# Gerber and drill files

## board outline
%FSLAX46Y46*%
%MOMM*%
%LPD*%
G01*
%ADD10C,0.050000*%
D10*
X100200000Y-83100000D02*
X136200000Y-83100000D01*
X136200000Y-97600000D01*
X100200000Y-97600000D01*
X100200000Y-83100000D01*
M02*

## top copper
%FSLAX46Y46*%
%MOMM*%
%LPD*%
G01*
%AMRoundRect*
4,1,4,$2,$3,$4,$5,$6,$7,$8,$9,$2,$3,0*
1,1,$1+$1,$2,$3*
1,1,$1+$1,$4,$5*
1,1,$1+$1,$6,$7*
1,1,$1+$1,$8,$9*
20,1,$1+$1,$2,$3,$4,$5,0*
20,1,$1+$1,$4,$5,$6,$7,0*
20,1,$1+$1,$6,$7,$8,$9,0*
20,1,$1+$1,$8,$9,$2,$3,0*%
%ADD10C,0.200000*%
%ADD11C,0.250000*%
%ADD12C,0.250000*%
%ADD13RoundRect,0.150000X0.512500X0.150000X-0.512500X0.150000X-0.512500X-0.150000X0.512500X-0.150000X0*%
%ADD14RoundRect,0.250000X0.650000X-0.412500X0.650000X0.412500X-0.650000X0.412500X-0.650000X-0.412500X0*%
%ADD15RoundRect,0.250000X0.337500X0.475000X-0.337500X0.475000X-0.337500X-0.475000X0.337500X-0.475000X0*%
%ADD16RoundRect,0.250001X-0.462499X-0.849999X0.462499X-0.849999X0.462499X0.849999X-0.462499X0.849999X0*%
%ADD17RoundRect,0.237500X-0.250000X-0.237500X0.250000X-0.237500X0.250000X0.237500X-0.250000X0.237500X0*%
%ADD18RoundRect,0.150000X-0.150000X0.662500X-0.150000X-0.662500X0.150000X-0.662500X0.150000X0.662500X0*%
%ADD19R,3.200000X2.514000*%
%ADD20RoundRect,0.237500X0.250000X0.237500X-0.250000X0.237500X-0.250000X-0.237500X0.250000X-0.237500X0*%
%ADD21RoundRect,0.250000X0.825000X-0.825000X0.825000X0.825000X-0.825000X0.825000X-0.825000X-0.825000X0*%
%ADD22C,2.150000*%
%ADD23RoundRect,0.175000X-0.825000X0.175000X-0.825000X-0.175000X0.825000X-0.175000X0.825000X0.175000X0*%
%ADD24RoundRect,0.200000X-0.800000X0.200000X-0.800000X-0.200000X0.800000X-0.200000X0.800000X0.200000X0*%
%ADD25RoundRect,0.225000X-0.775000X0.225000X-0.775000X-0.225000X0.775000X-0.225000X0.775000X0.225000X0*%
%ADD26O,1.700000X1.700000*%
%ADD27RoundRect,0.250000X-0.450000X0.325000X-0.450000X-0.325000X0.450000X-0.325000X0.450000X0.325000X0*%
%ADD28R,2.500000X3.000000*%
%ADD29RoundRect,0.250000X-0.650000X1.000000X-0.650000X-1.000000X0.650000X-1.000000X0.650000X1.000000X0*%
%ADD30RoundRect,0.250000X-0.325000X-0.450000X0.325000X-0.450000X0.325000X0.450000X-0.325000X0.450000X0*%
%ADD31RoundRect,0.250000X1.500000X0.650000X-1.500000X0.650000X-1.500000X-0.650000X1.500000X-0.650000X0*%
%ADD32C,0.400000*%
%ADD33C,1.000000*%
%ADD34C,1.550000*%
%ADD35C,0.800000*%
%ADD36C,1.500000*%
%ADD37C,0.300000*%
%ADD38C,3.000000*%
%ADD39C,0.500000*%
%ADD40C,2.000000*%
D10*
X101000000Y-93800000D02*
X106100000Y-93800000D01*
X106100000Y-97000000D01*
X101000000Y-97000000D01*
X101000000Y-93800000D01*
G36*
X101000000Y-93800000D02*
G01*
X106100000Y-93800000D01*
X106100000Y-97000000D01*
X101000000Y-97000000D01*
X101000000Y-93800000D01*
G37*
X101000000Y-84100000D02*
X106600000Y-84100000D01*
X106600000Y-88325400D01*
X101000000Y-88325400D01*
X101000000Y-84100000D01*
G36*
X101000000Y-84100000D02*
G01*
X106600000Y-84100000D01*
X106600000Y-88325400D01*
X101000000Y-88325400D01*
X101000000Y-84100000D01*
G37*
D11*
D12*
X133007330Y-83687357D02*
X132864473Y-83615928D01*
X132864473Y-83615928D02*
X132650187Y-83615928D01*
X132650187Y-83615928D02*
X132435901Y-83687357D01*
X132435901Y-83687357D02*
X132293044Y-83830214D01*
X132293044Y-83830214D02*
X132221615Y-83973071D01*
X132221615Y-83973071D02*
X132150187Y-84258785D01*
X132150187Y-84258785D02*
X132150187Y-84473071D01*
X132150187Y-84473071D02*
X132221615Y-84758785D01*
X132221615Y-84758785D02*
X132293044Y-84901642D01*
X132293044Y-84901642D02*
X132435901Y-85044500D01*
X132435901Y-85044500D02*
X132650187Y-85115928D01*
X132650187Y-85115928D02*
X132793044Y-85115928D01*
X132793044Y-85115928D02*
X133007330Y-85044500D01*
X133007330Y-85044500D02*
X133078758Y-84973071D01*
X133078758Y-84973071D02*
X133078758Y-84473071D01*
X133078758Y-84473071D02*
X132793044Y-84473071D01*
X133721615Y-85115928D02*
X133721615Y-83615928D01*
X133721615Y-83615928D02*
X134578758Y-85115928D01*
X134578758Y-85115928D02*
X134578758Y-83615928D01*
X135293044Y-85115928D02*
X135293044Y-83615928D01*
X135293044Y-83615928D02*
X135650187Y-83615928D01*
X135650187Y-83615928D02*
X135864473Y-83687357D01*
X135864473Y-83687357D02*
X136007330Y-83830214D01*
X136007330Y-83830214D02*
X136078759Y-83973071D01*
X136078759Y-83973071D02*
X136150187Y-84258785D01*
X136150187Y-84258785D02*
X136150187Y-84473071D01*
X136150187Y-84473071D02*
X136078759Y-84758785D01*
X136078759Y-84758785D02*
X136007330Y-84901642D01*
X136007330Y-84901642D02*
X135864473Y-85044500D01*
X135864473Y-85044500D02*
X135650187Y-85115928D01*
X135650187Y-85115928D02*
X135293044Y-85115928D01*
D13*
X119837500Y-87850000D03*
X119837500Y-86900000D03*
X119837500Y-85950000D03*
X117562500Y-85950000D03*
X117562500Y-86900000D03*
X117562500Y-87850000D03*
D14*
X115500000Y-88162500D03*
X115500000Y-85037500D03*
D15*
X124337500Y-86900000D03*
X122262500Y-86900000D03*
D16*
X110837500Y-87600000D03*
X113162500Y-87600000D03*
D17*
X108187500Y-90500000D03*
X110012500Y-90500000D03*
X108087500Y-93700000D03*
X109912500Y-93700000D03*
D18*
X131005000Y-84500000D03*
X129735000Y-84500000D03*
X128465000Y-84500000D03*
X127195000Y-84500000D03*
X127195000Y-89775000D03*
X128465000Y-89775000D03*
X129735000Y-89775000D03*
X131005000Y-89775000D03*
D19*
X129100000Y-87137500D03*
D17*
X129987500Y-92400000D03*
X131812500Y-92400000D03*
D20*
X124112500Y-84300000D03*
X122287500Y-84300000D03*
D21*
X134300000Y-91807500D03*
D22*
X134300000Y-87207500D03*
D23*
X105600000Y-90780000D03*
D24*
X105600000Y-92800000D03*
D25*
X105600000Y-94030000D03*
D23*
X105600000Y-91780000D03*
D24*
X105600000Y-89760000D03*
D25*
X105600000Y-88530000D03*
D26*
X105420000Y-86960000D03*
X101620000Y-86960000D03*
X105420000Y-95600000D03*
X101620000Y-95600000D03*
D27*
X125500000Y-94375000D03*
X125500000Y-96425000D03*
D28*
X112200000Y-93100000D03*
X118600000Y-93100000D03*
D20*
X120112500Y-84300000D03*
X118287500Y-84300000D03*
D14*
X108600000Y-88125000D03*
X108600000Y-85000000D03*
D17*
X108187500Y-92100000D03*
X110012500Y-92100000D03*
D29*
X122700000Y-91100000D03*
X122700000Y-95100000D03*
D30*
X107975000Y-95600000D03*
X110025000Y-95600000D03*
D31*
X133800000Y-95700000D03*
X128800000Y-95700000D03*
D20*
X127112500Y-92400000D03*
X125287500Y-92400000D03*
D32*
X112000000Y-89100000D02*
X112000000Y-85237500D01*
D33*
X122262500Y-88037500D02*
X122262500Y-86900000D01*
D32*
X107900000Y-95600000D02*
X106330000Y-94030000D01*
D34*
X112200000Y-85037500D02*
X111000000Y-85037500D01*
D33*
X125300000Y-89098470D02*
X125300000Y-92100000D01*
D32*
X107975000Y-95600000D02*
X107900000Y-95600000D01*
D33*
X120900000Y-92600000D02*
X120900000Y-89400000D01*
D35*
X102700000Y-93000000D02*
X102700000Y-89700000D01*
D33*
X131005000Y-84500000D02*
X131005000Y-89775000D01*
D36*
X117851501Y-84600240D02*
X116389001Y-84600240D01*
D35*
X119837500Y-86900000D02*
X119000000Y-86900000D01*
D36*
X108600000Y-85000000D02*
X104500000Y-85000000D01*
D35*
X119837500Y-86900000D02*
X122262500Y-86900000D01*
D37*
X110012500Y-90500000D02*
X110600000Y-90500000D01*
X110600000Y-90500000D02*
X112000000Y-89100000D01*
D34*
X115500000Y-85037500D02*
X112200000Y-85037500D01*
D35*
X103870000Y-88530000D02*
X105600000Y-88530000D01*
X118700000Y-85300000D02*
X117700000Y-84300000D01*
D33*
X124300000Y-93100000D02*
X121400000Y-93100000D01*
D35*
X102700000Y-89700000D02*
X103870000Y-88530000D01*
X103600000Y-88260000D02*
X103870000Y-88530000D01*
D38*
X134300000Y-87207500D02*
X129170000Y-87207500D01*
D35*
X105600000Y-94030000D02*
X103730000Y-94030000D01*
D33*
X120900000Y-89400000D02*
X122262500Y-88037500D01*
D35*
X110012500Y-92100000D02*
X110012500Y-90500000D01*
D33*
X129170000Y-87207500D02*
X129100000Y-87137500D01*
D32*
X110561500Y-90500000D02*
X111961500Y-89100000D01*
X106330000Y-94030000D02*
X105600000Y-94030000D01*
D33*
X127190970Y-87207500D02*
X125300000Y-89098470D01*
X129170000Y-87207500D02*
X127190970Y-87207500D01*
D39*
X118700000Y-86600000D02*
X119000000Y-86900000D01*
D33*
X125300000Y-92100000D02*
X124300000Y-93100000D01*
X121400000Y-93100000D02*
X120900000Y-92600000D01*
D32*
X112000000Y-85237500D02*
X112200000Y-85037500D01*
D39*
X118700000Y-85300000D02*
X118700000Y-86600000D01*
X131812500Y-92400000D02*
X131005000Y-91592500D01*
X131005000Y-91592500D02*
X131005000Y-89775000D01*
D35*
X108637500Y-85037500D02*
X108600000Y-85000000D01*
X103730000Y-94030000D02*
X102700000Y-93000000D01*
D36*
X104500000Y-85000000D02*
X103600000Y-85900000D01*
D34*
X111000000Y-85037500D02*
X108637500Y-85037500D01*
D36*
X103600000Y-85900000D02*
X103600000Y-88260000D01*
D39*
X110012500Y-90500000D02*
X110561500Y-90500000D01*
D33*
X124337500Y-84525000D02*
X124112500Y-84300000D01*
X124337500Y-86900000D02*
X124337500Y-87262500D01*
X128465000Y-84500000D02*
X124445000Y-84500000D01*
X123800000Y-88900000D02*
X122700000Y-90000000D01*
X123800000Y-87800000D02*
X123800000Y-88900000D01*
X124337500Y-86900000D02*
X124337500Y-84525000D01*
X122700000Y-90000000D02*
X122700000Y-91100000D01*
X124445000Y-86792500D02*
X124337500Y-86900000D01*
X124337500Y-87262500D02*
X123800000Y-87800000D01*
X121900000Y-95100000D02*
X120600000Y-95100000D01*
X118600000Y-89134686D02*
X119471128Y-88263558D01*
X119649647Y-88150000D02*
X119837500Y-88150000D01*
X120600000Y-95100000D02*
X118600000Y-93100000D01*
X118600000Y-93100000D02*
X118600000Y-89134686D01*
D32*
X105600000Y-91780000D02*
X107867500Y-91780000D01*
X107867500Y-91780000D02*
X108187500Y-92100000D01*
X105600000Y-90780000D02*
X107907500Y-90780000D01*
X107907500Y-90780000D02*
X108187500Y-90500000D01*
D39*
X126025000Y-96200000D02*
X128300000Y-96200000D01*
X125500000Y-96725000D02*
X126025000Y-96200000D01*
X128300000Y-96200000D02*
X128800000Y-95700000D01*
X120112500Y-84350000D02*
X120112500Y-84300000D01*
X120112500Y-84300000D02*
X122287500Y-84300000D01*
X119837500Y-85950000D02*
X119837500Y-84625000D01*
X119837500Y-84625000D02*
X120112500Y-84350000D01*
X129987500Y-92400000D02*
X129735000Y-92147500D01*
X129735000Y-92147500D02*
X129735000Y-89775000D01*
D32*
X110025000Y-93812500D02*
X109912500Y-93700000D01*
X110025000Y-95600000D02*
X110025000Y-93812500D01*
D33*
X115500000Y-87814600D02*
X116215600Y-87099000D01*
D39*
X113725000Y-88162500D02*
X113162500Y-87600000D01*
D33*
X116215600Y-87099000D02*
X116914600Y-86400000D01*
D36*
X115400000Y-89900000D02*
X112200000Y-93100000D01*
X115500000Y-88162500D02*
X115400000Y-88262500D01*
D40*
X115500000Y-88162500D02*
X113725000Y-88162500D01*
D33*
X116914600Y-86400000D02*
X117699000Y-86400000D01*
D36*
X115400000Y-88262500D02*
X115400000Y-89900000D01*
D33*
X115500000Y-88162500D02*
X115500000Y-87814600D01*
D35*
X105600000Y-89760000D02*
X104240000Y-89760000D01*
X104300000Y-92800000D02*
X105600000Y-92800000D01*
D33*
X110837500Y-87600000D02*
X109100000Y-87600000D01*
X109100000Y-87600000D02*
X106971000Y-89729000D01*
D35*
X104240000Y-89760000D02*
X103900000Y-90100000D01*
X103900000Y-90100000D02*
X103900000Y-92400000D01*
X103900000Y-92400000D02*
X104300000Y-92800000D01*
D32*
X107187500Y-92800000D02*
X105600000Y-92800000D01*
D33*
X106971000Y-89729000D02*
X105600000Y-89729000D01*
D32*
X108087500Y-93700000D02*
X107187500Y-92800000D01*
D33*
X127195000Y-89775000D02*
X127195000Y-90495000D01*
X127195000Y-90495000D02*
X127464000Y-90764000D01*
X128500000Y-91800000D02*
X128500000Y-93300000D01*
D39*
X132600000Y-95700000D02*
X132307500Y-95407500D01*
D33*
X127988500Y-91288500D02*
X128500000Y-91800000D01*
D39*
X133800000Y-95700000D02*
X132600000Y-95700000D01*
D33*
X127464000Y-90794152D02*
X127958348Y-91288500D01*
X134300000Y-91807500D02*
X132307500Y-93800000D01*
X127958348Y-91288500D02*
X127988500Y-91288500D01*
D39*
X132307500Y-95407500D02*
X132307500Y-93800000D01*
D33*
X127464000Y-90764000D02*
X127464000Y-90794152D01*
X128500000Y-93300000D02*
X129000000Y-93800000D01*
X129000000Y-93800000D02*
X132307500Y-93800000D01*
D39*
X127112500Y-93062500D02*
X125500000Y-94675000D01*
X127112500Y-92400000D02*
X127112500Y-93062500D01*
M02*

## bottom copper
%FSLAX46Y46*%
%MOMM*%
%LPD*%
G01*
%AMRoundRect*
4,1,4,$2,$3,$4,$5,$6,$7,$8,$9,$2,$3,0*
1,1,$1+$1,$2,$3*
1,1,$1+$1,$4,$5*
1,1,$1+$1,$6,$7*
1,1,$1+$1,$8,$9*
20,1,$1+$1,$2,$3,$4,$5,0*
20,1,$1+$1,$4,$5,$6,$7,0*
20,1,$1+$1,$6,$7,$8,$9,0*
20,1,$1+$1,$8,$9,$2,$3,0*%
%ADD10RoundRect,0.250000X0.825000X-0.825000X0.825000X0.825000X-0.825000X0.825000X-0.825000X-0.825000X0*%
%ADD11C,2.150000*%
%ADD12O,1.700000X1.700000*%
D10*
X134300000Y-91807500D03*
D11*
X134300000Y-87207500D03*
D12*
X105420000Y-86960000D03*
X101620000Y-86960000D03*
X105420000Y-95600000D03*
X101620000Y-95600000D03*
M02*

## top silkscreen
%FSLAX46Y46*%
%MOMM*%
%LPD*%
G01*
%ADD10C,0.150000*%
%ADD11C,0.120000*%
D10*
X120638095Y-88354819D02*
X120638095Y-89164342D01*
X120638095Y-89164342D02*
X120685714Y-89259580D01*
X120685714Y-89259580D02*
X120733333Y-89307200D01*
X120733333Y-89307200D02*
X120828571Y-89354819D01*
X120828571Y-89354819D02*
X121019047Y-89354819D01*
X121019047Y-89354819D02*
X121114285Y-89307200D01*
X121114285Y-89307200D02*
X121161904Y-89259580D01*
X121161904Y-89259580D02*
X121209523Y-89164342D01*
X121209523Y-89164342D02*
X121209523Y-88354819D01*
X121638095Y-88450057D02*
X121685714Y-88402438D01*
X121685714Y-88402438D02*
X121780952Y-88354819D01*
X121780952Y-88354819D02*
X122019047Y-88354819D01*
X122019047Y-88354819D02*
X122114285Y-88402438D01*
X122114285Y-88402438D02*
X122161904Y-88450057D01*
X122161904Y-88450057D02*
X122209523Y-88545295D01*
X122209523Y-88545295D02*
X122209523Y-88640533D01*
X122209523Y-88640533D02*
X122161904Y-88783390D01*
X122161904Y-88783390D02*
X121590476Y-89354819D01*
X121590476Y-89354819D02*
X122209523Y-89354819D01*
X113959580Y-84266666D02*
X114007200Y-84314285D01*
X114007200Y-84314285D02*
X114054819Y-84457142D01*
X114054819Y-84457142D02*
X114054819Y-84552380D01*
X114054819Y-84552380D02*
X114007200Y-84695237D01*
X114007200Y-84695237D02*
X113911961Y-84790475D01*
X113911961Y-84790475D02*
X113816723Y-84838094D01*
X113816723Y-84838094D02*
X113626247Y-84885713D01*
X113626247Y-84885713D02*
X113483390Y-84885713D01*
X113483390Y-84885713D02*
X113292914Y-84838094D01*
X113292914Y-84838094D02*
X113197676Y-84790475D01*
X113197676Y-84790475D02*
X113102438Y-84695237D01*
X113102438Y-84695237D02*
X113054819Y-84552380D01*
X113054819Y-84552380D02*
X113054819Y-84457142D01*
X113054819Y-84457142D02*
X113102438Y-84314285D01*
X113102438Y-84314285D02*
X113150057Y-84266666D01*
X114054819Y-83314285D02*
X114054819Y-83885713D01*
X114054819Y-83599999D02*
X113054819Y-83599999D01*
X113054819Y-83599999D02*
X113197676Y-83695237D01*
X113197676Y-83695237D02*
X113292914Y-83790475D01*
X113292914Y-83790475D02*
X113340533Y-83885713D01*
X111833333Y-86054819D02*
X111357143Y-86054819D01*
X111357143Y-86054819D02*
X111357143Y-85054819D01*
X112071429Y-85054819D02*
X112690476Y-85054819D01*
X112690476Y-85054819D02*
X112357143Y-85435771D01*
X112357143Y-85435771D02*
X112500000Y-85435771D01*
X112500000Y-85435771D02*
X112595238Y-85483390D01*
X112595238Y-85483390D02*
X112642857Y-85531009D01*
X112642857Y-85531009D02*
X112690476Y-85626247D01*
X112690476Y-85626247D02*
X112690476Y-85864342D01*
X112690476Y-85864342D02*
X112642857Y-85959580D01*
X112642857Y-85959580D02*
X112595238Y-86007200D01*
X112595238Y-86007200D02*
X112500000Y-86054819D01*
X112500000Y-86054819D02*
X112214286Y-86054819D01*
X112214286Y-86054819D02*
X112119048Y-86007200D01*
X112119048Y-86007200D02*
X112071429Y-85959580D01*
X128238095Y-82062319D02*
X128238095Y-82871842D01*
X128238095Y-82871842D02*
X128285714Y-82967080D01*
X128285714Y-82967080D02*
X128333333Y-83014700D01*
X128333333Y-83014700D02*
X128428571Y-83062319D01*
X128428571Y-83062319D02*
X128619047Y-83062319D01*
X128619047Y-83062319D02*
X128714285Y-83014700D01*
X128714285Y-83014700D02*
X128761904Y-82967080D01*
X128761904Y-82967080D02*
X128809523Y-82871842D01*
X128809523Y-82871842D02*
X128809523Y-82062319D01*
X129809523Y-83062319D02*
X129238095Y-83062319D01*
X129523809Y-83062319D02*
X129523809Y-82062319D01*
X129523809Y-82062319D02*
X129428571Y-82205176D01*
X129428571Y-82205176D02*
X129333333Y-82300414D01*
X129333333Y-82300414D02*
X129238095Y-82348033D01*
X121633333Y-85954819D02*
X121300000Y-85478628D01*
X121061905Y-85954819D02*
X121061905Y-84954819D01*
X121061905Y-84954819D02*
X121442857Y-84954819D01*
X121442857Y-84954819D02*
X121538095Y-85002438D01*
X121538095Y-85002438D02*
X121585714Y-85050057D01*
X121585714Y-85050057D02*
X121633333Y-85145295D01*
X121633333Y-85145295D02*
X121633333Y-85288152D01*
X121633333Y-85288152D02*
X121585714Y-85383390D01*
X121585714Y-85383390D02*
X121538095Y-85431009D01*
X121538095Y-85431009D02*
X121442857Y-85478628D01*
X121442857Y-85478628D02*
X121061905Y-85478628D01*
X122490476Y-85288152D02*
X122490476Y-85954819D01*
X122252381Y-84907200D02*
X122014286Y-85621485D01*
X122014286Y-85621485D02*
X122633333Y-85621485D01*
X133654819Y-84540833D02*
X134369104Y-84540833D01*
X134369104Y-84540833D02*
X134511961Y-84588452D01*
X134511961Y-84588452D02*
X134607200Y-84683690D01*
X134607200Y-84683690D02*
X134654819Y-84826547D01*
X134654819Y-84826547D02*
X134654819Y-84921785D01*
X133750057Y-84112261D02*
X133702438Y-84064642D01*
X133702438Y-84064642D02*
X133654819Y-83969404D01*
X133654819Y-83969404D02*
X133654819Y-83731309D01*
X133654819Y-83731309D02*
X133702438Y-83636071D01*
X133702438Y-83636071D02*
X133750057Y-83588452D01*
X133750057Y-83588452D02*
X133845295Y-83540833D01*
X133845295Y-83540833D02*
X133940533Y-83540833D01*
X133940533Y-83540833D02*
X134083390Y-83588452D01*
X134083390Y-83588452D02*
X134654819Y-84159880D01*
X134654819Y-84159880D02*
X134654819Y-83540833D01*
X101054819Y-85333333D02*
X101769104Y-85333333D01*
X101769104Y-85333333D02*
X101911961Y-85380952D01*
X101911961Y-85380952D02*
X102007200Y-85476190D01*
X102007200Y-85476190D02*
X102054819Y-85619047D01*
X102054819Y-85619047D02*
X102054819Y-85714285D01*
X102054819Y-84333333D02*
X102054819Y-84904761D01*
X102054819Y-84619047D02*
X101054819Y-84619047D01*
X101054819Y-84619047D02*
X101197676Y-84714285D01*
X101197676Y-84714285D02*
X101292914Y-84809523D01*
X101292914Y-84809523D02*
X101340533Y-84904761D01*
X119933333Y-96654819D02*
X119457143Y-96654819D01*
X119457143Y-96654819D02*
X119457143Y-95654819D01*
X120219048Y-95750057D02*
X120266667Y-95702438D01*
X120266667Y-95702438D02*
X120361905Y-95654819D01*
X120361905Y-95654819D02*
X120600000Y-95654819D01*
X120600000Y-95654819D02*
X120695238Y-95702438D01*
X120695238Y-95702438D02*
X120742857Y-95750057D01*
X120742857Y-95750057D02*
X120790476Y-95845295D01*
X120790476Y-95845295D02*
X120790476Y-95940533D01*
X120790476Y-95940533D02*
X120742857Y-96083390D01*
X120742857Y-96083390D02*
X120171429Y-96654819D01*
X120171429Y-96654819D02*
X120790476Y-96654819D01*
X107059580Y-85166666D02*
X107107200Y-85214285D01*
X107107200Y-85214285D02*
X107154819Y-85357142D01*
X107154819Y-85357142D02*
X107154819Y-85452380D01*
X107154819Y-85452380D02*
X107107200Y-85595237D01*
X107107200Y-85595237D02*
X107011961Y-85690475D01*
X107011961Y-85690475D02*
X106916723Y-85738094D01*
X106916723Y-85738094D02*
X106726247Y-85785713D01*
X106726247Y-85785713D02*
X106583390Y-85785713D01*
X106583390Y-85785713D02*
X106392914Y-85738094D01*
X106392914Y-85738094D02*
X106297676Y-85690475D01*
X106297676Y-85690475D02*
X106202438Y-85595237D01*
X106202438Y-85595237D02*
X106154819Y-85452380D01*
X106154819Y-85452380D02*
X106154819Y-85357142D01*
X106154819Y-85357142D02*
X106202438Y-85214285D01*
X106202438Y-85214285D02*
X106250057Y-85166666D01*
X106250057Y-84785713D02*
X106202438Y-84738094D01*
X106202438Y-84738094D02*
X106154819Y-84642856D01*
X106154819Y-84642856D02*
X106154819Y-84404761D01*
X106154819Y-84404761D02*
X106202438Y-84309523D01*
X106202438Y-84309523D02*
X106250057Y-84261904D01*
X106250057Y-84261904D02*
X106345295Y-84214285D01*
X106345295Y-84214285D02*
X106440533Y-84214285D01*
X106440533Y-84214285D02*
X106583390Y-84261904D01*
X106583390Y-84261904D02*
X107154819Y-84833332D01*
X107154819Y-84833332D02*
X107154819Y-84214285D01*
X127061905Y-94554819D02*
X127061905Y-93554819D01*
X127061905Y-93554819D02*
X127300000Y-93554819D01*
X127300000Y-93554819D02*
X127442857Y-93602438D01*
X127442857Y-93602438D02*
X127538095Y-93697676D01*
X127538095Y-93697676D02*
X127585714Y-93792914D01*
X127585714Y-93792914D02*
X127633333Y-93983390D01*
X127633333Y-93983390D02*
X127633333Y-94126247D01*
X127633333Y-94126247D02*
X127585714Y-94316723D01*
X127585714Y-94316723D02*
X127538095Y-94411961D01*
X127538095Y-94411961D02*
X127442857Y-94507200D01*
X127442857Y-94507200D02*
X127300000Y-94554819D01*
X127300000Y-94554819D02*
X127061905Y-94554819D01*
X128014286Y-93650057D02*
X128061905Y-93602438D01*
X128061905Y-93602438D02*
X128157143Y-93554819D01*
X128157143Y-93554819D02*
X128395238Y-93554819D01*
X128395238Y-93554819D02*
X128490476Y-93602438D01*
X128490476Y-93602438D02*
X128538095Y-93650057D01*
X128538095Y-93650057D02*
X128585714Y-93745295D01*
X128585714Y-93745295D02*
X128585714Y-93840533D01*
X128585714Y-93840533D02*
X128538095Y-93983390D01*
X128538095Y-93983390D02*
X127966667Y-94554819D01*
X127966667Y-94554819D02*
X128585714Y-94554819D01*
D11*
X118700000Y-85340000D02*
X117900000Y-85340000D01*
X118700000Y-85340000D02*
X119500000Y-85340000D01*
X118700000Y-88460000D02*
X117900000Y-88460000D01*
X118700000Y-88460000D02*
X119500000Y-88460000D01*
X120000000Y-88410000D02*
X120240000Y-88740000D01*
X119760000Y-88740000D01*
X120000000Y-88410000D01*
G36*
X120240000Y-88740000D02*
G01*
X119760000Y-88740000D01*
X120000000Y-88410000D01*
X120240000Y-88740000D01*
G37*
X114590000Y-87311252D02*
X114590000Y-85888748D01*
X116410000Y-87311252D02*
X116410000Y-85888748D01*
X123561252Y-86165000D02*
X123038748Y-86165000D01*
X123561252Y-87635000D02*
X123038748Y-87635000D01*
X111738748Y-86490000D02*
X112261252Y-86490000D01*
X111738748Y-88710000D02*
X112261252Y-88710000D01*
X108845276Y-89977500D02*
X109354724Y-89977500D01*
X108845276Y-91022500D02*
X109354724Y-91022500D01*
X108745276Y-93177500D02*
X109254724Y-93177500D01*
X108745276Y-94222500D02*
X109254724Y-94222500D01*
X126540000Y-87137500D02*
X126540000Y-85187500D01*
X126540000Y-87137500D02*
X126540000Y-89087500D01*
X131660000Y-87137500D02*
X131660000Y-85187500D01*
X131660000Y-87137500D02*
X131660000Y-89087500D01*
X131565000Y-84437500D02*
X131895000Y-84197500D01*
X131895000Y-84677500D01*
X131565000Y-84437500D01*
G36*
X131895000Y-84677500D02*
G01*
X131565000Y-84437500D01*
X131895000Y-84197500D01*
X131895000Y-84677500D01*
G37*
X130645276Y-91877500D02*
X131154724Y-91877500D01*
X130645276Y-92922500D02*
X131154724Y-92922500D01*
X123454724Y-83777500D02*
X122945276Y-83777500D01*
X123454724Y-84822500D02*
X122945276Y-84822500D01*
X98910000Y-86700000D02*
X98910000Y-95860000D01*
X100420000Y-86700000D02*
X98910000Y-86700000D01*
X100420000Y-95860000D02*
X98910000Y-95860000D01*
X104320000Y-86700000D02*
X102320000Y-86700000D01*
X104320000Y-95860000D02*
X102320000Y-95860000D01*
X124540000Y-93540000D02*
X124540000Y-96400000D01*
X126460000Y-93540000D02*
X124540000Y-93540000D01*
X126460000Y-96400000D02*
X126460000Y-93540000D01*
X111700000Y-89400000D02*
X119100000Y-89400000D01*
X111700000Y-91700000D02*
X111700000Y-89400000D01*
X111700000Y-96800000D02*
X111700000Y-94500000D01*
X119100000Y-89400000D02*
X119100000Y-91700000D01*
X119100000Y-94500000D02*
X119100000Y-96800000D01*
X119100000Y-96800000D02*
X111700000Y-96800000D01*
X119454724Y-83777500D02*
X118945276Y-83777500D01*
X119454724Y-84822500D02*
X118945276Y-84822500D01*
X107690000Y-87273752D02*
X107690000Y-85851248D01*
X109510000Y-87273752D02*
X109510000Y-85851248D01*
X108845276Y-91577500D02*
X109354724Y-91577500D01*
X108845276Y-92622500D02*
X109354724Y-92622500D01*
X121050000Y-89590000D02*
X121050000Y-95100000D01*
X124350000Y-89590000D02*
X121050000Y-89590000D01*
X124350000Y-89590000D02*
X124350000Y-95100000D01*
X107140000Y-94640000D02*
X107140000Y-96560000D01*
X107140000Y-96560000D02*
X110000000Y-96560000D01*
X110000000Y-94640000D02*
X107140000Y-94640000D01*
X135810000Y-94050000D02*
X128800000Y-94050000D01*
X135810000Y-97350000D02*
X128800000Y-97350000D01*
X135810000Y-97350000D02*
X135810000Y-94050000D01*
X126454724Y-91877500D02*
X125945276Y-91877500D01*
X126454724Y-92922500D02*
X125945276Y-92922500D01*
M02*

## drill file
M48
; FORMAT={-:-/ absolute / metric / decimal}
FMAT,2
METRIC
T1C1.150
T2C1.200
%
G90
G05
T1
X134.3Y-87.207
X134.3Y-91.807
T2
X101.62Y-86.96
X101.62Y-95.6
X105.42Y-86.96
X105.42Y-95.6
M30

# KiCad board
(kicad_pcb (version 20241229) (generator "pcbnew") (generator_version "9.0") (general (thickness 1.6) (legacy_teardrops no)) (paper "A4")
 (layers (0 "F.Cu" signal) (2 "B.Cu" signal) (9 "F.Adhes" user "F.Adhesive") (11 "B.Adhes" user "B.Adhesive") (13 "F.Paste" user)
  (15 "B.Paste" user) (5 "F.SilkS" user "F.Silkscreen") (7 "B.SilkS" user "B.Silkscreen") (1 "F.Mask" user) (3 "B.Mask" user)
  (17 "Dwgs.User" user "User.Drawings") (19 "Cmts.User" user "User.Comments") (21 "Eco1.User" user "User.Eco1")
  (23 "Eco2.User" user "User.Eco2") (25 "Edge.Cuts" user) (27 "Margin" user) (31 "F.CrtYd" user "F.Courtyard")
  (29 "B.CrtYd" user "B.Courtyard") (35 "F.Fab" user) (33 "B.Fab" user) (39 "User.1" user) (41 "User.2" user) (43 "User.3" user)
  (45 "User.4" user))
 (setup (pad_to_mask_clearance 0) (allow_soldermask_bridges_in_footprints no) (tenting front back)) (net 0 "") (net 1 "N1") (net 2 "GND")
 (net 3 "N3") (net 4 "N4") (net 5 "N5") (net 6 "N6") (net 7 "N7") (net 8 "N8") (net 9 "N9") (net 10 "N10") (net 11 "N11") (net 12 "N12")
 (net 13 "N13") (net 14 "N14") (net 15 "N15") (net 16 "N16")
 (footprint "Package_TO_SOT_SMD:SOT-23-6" (layer "F.Cu") (at 118.7 86.9 180)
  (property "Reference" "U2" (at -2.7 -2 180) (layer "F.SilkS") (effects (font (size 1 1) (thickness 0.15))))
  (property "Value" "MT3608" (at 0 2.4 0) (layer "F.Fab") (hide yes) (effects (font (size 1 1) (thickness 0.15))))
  (fp_line (start 0 1.56) (end 0.8 1.56) (stroke (width 0.12) (type solid)) (layer "F.SilkS"))
  (fp_line (start 0 1.56) (end -0.8 1.56) (stroke (width 0.12) (type solid)) (layer "F.SilkS"))
  (fp_line (start 0 -1.56) (end 0.8 -1.56) (stroke (width 0.12) (type solid)) (layer "F.SilkS"))
  (fp_line (start 0 -1.56) (end -0.8 -1.56) (stroke (width 0.12) (type solid)) (layer "F.SilkS"))
  (fp_poly (pts (xy -1.3 -1.51) (xy -1.54 -1.84) (xy -1.06 -1.84)) (stroke (width 0.12) (type solid)) (fill yes) (layer "F.SilkS"))
  (pad "1" smd roundrect (at -1.1375 -0.95 180) (size 1.325 0.6) (layers "F.Cu" "F.Mask" "F.Paste") (roundrect_rratio 0.25) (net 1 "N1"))
  (pad "2" smd roundrect (at -1.1375 0 180) (size 1.325 0.6) (layers "F.Cu" "F.Mask" "F.Paste") (roundrect_rratio 0.25) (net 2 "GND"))
  (pad "3" smd roundrect (at -1.1375 0.95 180) (size 1.325 0.6) (layers "F.Cu" "F.Mask" "F.Paste") (roundrect_rratio 0.25) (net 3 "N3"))
  (pad "4" smd roundrect (at 1.1375 0.95 180) (size 1.325 0.6) (layers "F.Cu" "F.Mask" "F.Paste") (roundrect_rratio 0.25) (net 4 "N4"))
  (pad "5" smd roundrect (at 1.1375 0 180) (size 1.325 0.6) (layers "F.Cu" "F.Mask" "F.Paste") (roundrect_rratio 0.25) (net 4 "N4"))
  (pad "6" smd roundrect (at 1.1375 -0.95 180) (size 1.325 0.6) (layers "F.Cu" "F.Mask" "F.Paste") (roundrect_rratio 0.25) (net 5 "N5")))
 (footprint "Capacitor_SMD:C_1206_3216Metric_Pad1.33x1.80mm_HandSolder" (layer "F.Cu") (at 115.5 86.6 90)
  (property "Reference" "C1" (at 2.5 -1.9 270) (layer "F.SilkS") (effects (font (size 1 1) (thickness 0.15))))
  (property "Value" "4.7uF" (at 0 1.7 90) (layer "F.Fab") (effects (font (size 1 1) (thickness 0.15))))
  (fp_line (start -0.711252 -0.91) (end 0.711252 -0.91) (stroke (width 0.12) (type solid)) (layer "F.SilkS"))
  (fp_line (start -0.711252 0.91) (end 0.711252 0.91) (stroke (width 0.12) (type solid)) (layer "F.SilkS"))
  (pad "1" smd roundrect (at -1.5625 0 90) (size 1.325 1.8) (layers "F.Cu" "F.Mask" "F.Paste") (roundrect_rratio 0.188679) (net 4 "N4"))
  (pad "2" smd roundrect (at 1.5625 0 90) (size 1.325 1.8) (layers "F.Cu" "F.Mask" "F.Paste") (roundrect_rratio 0.188679) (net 2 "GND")))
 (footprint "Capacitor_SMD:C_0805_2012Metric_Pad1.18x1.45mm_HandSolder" (layer "F.Cu") (at 123.3 86.9 180)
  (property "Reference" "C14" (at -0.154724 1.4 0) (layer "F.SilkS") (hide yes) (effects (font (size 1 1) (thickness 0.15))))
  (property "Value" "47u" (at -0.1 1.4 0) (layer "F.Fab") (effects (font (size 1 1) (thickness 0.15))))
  (fp_line (start -0.261252 0.735) (end 0.261252 0.735) (stroke (width 0.12) (type solid)) (layer "F.SilkS"))
  (fp_line (start -0.261252 -0.735) (end 0.261252 -0.735) (stroke (width 0.12) (type solid)) (layer "F.SilkS"))
  (pad "1" smd roundrect (at -1.0375 0 180) (size 1.175 1.45) (layers "F.Cu" "F.Mask" "F.Paste") (roundrect_rratio 0.212766) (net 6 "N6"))
  (pad "2" smd roundrect (at 1.0375 0 180) (size 1.175 1.45) (layers "F.Cu" "F.Mask" "F.Paste") (roundrect_rratio 0.212766) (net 2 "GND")))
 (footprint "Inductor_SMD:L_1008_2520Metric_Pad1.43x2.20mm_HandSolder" (layer "F.Cu") (at 112 87.6)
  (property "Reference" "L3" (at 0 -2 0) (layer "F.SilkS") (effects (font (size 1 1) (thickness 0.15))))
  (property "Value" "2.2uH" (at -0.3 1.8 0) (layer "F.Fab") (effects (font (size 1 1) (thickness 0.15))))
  (fp_line (start -0.261252 -1.11) (end 0.261252 -1.11) (stroke (width 0.12) (type solid)) (layer "F.SilkS"))
  (fp_line (start -0.261252 1.11) (end 0.261252 1.11) (stroke (width 0.12) (type solid)) (layer "F.SilkS"))
  (pad "1" smd roundrect (at -1.1625 0) (size 1.425 2.2) (layers "F.Cu" "F.Mask" "F.Paste") (roundrect_rratio 0.175439) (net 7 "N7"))
  (pad "2" smd roundrect (at 1.1625 0) (size 1.425 2.2) (layers "F.Cu" "F.Mask" "F.Paste") (roundrect_rratio 0.175439) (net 4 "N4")))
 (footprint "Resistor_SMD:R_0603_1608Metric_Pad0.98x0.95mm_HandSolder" (layer "F.Cu") (at 109.1 90.5)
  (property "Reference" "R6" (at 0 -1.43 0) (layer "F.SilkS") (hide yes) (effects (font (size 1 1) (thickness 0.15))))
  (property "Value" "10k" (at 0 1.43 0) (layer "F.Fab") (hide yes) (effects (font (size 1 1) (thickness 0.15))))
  (fp_line (start -0.254724 -0.5225) (end 0.254724 -0.5225) (stroke (width 0.12) (type solid)) (layer "F.SilkS"))
  (fp_line (start -0.254724 0.5225) (end 0.254724 0.5225) (stroke (width 0.12) (type solid)) (layer "F.SilkS"))
  (pad "1" smd roundrect (at -0.9125 0) (size 0.975 0.95) (layers "F.Cu" "F.Mask" "F.Paste") (roundrect_rratio 0.25) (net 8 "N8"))
  (pad "2" smd roundrect (at 0.9125 0) (size 0.975 0.95) (layers "F.Cu" "F.Mask" "F.Paste") (roundrect_rratio 0.25) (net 2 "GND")))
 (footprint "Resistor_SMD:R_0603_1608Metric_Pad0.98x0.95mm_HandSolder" (layer "F.Cu") (at 109 93.7)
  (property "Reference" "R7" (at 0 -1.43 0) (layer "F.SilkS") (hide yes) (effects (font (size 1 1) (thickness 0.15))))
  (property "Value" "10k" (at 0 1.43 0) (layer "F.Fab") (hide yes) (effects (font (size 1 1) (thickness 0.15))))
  (fp_line (start -0.254724 -0.5225) (end 0.254724 -0.5225) (stroke (width 0.12) (type solid)) (layer "F.SilkS"))
  (fp_line (start -0.254724 0.5225) (end 0.254724 0.5225) (stroke (width 0.12) (type solid)) (layer "F.SilkS"))
  (pad "1" smd roundrect (at -0.9125 0) (size 0.975 0.95) (layers "F.Cu" "F.Mask" "F.Paste") (roundrect_rratio 0.25) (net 7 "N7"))
  (pad "2" smd roundrect (at 0.9125 0) (size 0.975 0.95) (layers "F.Cu" "F.Mask" "F.Paste") (roundrect_rratio 0.25) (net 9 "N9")))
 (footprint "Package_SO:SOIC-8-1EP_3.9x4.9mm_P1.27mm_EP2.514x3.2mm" (layer "F.Cu") (at 129.1 87.1375 -90)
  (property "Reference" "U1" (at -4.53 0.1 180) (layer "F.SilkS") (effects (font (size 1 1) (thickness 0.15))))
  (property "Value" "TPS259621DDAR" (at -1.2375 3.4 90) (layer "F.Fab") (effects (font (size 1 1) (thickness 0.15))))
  (fp_line (start 0 2.56) (end -1.95 2.56) (stroke (width 0.12) (type solid)) (layer "F.SilkS"))
  (fp_line (start 0 2.56) (end 1.95 2.56) (stroke (width 0.12) (type solid)) (layer "F.SilkS"))
  (fp_line (start 0 -2.56) (end -1.95 -2.56) (stroke (width 0.12) (type solid)) (layer "F.SilkS"))
  (fp_line (start 0 -2.56) (end 1.95 -2.56) (stroke (width 0.12) (type solid)) (layer "F.SilkS"))
  (fp_poly (pts (xy -2.7 -2.465) (xy -2.94 -2.795) (xy -2.46 -2.795)) (stroke (width 0.12) (type solid)) (fill yes) (layer "F.SilkS"))
  (pad "" smd roundrect (at -0.63 -0.8 270) (size 1.01 1.29) (layers "F.Paste") (roundrect_rratio 0.247525))
  (pad "" smd roundrect (at -0.63 0.8 270) (size 1.01 1.29) (layers "F.Paste") (roundrect_rratio 0.247525))
  (pad "" smd roundrect (at 0.63 -0.8 270) (size 1.01 1.29) (layers "F.Paste") (roundrect_rratio 0.247525))
  (pad "" smd roundrect (at 0.63 0.8 270) (size 1.01 1.29) (layers "F.Paste") (roundrect_rratio 0.247525))
  (pad "1" smd roundrect (at -2.6375 -1.905 270) (size 1.625 0.6) (layers "F.Cu" "F.Mask" "F.Paste") (roundrect_rratio 0.25) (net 2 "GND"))
  (pad "2" smd roundrect (at -2.6375 -0.635 270) (size 1.625 0.6) (layers "F.Cu" "F.Mask" "F.Paste") (roundrect_rratio 0.25) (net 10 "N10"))
  (pad "3" smd roundrect (at -2.6375 0.635 270) (size 1.625 0.6) (layers "F.Cu" "F.Mask" "F.Paste") (roundrect_rratio 0.25) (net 6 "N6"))
  (pad "4" smd roundrect (at -2.6375 1.905 270) (size 1.625 0.6) (layers "F.Cu" "F.Mask" "F.Paste") (roundrect_rratio 0.25) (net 6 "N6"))
  (pad "5" smd roundrect (at 2.6375 1.905 270) (size 1.625 0.6) (layers "F.Cu" "F.Mask" "F.Paste") (roundrect_rratio 0.25) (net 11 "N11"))
  (pad "6" smd roundrect (at 2.6375 0.635 270) (size 1.625 0.6) (layers "F.Cu" "F.Mask" "F.Paste") (roundrect_rratio 0.25) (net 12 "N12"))
  (pad "7" smd roundrect (at 2.6375 -0.635 270) (size 1.625 0.6) (layers "F.Cu" "F.Mask" "F.Paste") (roundrect_rratio 0.25) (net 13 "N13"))
  (pad "8" smd roundrect (at 2.6375 -1.905 270) (size 1.625 0.6) (layers "F.Cu" "F.Mask" "F.Paste") (roundrect_rratio 0.25) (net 2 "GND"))
  (pad "9" smd rect (at 0 0 270) (size 2.514 3.2) (layers "F.Cu" "F.Mask") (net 2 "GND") (zone_connect 2)))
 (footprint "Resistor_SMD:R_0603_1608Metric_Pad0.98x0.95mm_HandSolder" (layer "F.Cu") (at 130.9 92.4)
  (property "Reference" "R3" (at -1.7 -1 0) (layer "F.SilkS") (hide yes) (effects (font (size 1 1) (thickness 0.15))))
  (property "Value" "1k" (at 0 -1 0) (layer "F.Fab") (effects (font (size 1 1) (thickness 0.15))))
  (fp_line (start -0.254724 -0.5225) (end 0.254724 -0.5225) (stroke (width 0.12) (type solid)) (layer "F.SilkS"))
  (fp_line (start -0.254724 0.5225) (end 0.254724 0.5225) (stroke (width 0.12) (type solid)) (layer "F.SilkS"))
  (pad "1" smd roundrect (at -0.9125 0) (size 0.975 0.95) (layers "F.Cu" "F.Mask" "F.Paste") (roundrect_rratio 0.25) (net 13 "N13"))
  (pad "2" smd roundrect (at 0.9125 0) (size 0.975 0.95) (layers "F.Cu" "F.Mask" "F.Paste") (roundrect_rratio 0.25) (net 2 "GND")))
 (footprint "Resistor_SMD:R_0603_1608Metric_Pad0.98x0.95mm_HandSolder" (layer "F.Cu") (at 123.2 84.3 180)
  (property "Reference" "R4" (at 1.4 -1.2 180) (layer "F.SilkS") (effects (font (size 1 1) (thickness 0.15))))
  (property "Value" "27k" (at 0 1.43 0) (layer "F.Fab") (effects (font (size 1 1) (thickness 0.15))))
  (fp_line (start -0.254724 0.5225) (end 0.254724 0.5225) (stroke (width 0.12) (type solid)) (layer "F.SilkS"))
  (fp_line (start -0.254724 -0.5225) (end 0.254724 -0.5225) (stroke (width 0.12) (type solid)) (layer "F.SilkS"))
  (pad "1" smd roundrect (at -0.9125 0 180) (size 0.975 0.95) (layers "F.Cu" "F.Mask" "F.Paste") (roundrect_rratio 0.25) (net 6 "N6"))
  (pad "2" smd roundrect (at 0.9125 0 180) (size 0.975 0.95) (layers "F.Cu" "F.Mask" "F.Paste") (roundrect_rratio 0.25) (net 3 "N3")))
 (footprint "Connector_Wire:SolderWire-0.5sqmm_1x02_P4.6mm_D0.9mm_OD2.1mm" (layer "F.Cu") (at 134.3 91.8075 90)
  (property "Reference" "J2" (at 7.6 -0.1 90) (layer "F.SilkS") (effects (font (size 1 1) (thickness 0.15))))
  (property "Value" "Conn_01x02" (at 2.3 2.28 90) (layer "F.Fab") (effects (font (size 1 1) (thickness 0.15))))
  (pad "1" thru_hole roundrect (at 0 0 90) (size 2.15 2.15) (drill 1.15) (layers "*.Cu" "*.Mask") (remove_unused_layers no)
   (roundrect_rratio 0.116279) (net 11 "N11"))
  (pad "2" thru_hole circle (at 4.6 0 90) (size 2.15 2.15) (drill 1.15) (layers "*.Cu" "*.Mask") (remove_unused_layers no) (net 2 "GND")))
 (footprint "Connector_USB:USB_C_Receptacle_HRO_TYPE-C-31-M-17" (layer "F.Cu") (at 102.42 91.28 -90)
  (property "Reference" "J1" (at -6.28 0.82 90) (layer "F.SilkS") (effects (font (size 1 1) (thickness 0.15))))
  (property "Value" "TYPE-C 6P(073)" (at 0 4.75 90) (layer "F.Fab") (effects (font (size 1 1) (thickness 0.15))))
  (fp_line (start -4.58 3.51) (end 4.58 3.51) (stroke (width 0.12) (type solid)) (layer "F.SilkS"))
  (fp_line (start -4.58 2) (end -4.58 3.51) (stroke (width 0.12) (type solid)) (layer "F.SilkS"))
  (fp_line (start 4.58 2) (end 4.58 3.51) (stroke (width 0.12) (type solid)) (layer "F.SilkS"))
  (fp_line (start -4.58 -1.9) (end -4.58 0.1) (stroke (width 0.12) (type solid)) (layer "F.SilkS"))
  (fp_line (start 4.58 -1.9) (end 4.58 0.1) (stroke (width 0.12) (type solid)) (layer "F.SilkS"))
  (pad "A5" smd roundrect (at -0.5 -3.18 270) (size 0.7 2) (layers "F.Cu" "F.Mask" "F.Paste") (roundrect_rratio 0.25) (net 8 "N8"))
  (pad "A9" smd roundrect (at 1.52 -3.18 270) (size 0.8 2) (layers "F.Cu" "F.Mask" "F.Paste") (roundrect_rratio 0.25) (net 7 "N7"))
  (pad "A12" smd roundrect (at 2.75 -3.18 270) (size 0.9 2) (layers "F.Cu" "F.Mask" "F.Paste") (roundrect_rratio 0.25) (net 2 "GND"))
  (pad "B5" smd roundrect (at 0.5 -3.18 270) (size 0.7 2) (layers "F.Cu" "F.Mask" "F.Paste") (roundrect_rratio 0.25) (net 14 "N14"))
  (pad "B9" smd roundrect (at -1.52 -3.18 270) (size 0.8 2) (layers "F.Cu" "F.Mask" "F.Paste") (roundrect_rratio 0.25) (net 7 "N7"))
  (pad "B12" smd roundrect (at -2.75 -3.18 270) (size 0.9 2) (layers "F.Cu" "F.Mask" "F.Paste") (roundrect_rratio 0.25) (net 2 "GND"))
  (pad "S1" thru_hole oval (at -4.32 -3 270) (size 1.7 1.7) (drill oval 1.2) (layers "*.Cu" "*.Mask") (remove_unused_layers no)
   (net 2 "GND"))
  (pad "S1" thru_hole oval (at -4.32 0.8 270) (size 1.7 1.7) (drill oval 1.2) (layers "*.Cu" "*.Mask") (remove_unused_layers no)
   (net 2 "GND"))
  (pad "S1" thru_hole oval (at 4.32 -3 270) (size 1.7 1.7) (drill oval 1.2) (layers "*.Cu" "*.Mask") (remove_unused_layers no) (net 2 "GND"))
  (pad "S1" thru_hole oval (at 4.32 0.8 270) (size 1.7 1.7) (drill oval 1.2) (layers "*.Cu" "*.Mask") (remove_unused_layers no)
   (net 2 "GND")))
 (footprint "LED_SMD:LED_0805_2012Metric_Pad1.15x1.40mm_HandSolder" (layer "F.Cu") (at 125.5 95.4 -90)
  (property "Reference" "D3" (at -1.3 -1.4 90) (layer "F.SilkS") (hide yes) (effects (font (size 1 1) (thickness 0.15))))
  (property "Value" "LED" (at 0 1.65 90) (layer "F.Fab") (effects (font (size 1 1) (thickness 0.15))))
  (fp_line (start -1.86 0.96) (end 1 0.96) (stroke (width 0.12) (type solid)) (layer "F.SilkS"))
  (fp_line (start -1.86 -0.96) (end -1.86 0.96) (stroke (width 0.12) (type solid)) (layer "F.SilkS"))
  (fp_line (start 1 -0.96) (end -1.86 -0.96) (stroke (width 0.12) (type solid)) (layer "F.SilkS"))
  (pad "1" smd roundrect (at -1.025 0 270) (size 1.15 1.4) (layers "F.Cu" "F.Mask" "F.Paste") (roundrect_rratio 0.217391) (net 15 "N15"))
  (pad "2" smd roundrect (at 1.025 0 270) (size 1.15 1.4) (layers "F.Cu" "F.Mask" "F.Paste") (roundrect_rratio 0.217391) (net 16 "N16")))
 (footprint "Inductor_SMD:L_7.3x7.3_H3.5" (layer "F.Cu") (at 115.4 93.1)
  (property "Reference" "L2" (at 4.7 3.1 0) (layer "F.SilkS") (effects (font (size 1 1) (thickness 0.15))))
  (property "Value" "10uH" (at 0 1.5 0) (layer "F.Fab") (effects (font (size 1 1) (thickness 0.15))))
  (fp_line (start -3.7 -3.7) (end 3.7 -3.7) (stroke (width 0.12) (type solid)) (layer "F.SilkS"))
  (fp_line (start -3.7 -1.4) (end -3.7 -3.7) (stroke (width 0.12) (type solid)) (layer "F.SilkS"))
  (fp_line (start -3.7 3.7) (end -3.7 1.4) (stroke (width 0.12) (type solid)) (layer "F.SilkS"))
  (fp_line (start 3.7 -3.7) (end 3.7 -1.4) (stroke (width 0.12) (type solid)) (layer "F.SilkS"))
  (fp_line (start 3.7 1.4) (end 3.7 3.7) (stroke (width 0.12) (type solid)) (layer "F.SilkS"))
  (fp_line (start 3.7 3.7) (end -3.7 3.7) (stroke (width 0.12) (type solid)) (layer "F.SilkS"))
  (pad "1" smd rect (at -3.2 0) (size 2.5 3) (layers "F.Cu" "F.Mask" "F.Paste") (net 4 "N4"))
  (pad "2" smd rect (at 3.2 0) (size 2.5 3) (layers "F.Cu" "F.Mask" "F.Paste") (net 1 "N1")))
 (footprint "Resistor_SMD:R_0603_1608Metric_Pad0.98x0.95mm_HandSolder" (layer "F.Cu") (at 119.2 84.3 180)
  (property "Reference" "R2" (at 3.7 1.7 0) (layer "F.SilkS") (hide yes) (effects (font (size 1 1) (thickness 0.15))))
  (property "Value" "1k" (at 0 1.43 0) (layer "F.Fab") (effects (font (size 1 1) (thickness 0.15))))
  (fp_line (start -0.254724 0.5225) (end 0.254724 0.5225) (stroke (width 0.12) (type solid)) (layer "F.SilkS"))
  (fp_line (start -0.254724 -0.5225) (end 0.254724 -0.5225) (stroke (width 0.12) (type solid)) (layer "F.SilkS"))
  (pad "1" smd roundrect (at -0.9125 0 180) (size 0.975 0.95) (layers "F.Cu" "F.Mask" "F.Paste") (roundrect_rratio 0.25) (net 3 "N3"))
  (pad "2" smd roundrect (at 0.9125 0 180) (size 0.975 0.95) (layers "F.Cu" "F.Mask" "F.Paste") (roundrect_rratio 0.25) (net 2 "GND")))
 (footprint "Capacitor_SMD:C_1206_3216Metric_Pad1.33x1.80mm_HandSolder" (layer "F.Cu") (at 108.6 86.5625 90)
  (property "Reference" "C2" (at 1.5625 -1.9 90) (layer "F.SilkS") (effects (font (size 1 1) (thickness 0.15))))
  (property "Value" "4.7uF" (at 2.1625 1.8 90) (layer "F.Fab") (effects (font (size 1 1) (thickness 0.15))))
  (fp_line (start -0.711252 -0.91) (end 0.711252 -0.91) (stroke (width 0.12) (type solid)) (layer "F.SilkS"))
  (fp_line (start -0.711252 0.91) (end 0.711252 0.91) (stroke (width 0.12) (type solid)) (layer "F.SilkS"))
  (pad "1" smd roundrect (at -1.5625 0 90) (size 1.325 1.8) (layers "F.Cu" "F.Mask" "F.Paste") (roundrect_rratio 0.188679) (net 7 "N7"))
  (pad "2" smd roundrect (at 1.5625 0 90) (size 1.325 1.8) (layers "F.Cu" "F.Mask" "F.Paste") (roundrect_rratio 0.188679) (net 2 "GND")))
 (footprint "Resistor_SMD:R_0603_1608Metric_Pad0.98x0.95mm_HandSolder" (layer "F.Cu") (at 109.1 92.1)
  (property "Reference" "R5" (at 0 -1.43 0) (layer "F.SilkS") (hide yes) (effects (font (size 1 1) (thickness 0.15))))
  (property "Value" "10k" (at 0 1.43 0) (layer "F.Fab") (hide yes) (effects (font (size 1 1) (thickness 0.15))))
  (fp_line (start -0.254724 -0.5225) (end 0.254724 -0.5225) (stroke (width 0.12) (type solid)) (layer "F.SilkS"))
  (fp_line (start -0.254724 0.5225) (end 0.254724 0.5225) (stroke (width 0.12) (type solid)) (layer "F.SilkS"))
  (pad "1" smd roundrect (at -0.9125 0) (size 0.975 0.95) (layers "F.Cu" "F.Mask" "F.Paste") (roundrect_rratio 0.25) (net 14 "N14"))
  (pad "2" smd roundrect (at 0.9125 0) (size 0.975 0.95) (layers "F.Cu" "F.Mask" "F.Paste") (roundrect_rratio 0.25) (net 2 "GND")))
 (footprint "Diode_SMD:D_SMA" (layer "F.Cu") (at 122.7 93.1 -90)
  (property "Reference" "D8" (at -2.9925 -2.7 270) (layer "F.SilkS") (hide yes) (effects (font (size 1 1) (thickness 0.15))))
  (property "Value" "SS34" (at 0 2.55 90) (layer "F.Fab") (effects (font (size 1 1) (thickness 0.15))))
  (fp_line (start -3.51 1.65) (end 2 1.65) (stroke (width 0.12) (type solid)) (layer "F.SilkS"))
  (fp_line (start -3.51 -1.65) (end -3.51 1.65) (stroke (width 0.12) (type solid)) (layer "F.SilkS"))
  (fp_line (start -3.51 -1.65) (end 2 -1.65) (stroke (width 0.12) (type solid)) (layer "F.SilkS"))
  (pad "1" smd roundrect (at -2 0 270) (size 2.5 1.8) (layers "F.Cu" "F.Mask" "F.Paste") (roundrect_rratio 0.1388888889) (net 6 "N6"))
  (pad "2" smd roundrect (at 2 0 270) (size 2.5 1.8) (layers "F.Cu" "F.Mask" "F.Paste") (roundrect_rratio 0.1388888889) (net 1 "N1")))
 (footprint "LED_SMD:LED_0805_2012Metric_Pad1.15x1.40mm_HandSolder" (layer "F.Cu") (at 109 95.6)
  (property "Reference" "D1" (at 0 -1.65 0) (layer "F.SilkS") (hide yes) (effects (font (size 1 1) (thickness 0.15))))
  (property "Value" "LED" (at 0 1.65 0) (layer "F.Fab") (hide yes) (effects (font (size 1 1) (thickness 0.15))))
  (fp_line (start -1.86 -0.96) (end -1.86 0.96) (stroke (width 0.12) (type solid)) (layer "F.SilkS"))
  (fp_line (start -1.86 0.96) (end 1 0.96) (stroke (width 0.12) (type solid)) (layer "F.SilkS"))
  (fp_line (start 1 -0.96) (end -1.86 -0.96) (stroke (width 0.12) (type solid)) (layer "F.SilkS"))
  (pad "1" smd roundrect (at -1.025 0) (size 1.15 1.4) (layers "F.Cu" "F.Mask" "F.Paste") (roundrect_rratio 0.217391) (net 2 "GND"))
  (pad "2" smd roundrect (at 1.025 0) (size 1.15 1.4) (layers "F.Cu" "F.Mask" "F.Paste") (roundrect_rratio 0.217391) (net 9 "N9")))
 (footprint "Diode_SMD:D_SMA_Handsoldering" (layer "F.Cu") (at 131.3 95.7 180)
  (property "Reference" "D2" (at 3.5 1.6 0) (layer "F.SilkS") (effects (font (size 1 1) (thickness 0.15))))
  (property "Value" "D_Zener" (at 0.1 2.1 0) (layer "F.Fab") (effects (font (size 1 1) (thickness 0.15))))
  (fp_line (start -4.51 1.65) (end 2.5 1.65) (stroke (width 0.12) (type solid)) (layer "F.SilkS"))
  (fp_line (start -4.51 -1.65) (end 2.5 -1.65) (stroke (width 0.12) (type solid)) (layer "F.SilkS"))
  (fp_line (start -4.51 -1.65) (end -4.51 1.65) (stroke (width 0.12) (type solid)) (layer "F.SilkS"))
  (pad "1" smd roundrect (at -2.5 0 180) (size 3.5 1.8) (layers "F.Cu" "F.Mask" "F.Paste") (roundrect_rratio 0.1388888889) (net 11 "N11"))
  (pad "2" smd roundrect (at 2.5 0 180) (size 3.5 1.8) (layers "F.Cu" "F.Mask" "F.Paste") (roundrect_rratio 0.1388888889) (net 16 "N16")))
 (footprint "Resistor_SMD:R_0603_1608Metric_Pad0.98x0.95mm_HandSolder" (layer "F.Cu") (at 126.2 92.4 180)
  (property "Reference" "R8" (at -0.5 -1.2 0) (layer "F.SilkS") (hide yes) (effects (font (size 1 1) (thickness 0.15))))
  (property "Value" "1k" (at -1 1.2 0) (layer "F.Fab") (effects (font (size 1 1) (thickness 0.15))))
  (fp_line (start -0.254724 0.5225) (end 0.254724 0.5225) (stroke (width 0.12) (type solid)) (layer "F.SilkS"))
  (fp_line (start -0.254724 -0.5225) (end 0.254724 -0.5225) (stroke (width 0.12) (type solid)) (layer "F.SilkS"))
  (pad "1" smd roundrect (at -0.9125 0 180) (size 0.975 0.95) (layers "F.Cu" "F.Mask" "F.Paste") (roundrect_rratio 0.25) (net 15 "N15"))
  (pad "2" smd roundrect (at 0.9125 0 180) (size 0.975 0.95) (layers "F.Cu" "F.Mask" "F.Paste") (roundrect_rratio 0.25) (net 2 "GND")))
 (gr_rect (start 101 93.8) (end 106.1 97) (stroke (width 0.2) (type solid)) (fill yes) (layer "F.Cu") (net 2))
 (gr_rect (start 101 84.1) (end 106.6 88.3254) (stroke (width 0.2) (type solid)) (fill yes) (layer "F.Cu") (net 2))
 (gr_rect (start 100.2 83.1) (end 136.2 97.6) (stroke (width 0.05) (type default)) (fill no) (layer "Edge.Cuts"))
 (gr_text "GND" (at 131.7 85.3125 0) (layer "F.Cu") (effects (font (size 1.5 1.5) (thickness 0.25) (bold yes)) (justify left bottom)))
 (segment (start 112 89.1) (end 112 85.2375) (width 0.4) (layer "F.Cu") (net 2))
 (segment (start 122.2625 88.0375) (end 122.2625 86.9) (width 1) (layer "F.Cu") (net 2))
 (segment (start 107.9 95.6) (end 106.33 94.03) (width 0.4) (layer "F.Cu") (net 2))
 (segment (start 112.2 85.0375) (end 111 85.0375) (width 1.55) (layer "F.Cu") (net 2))
 (segment (start 125.3 89.09847) (end 125.3 92.1) (width 1) (layer "F.Cu") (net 2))
 (segment (start 107.975 95.6) (end 107.9 95.6) (width 0.4) (layer "F.Cu") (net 2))
 (segment (start 120.9 92.6) (end 120.9 89.4) (width 1) (layer "F.Cu") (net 2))
 (segment (start 102.7 93) (end 102.7 89.7) (width 0.8) (layer "F.Cu") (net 2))
 (segment (start 131.005 84.5) (end 131.005 89.775) (width 1) (layer "F.Cu") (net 2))
 (segment (start 117.851501 84.60024) (end 116.389001 84.60024) (width 1.5) (layer "F.Cu") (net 2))
 (segment (start 119.8375 86.9) (end 119 86.9) (width 0.8) (layer "F.Cu") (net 2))
 (segment (start 108.6 85) (end 104.5 85) (width 1.5) (layer "F.Cu") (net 2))
 (segment (start 119.8375 86.9) (end 122.2625 86.9) (width 0.8) (layer "F.Cu") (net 2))
 (segment (start 110.0125 90.5) (end 110.6 90.5) (width 0.3) (layer "F.Cu") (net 2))
 (segment (start 110.6 90.5) (end 112 89.1) (width 0.3) (layer "F.Cu") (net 2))
 (segment (start 115.5 85.0375) (end 112.2 85.0375) (width 1.55) (layer "F.Cu") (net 2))
 (segment (start 103.87 88.53) (end 105.6 88.53) (width 0.8) (layer "F.Cu") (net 2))
 (segment (start 118.7 85.3) (end 117.7 84.3) (width 0.8) (layer "F.Cu") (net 2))
 (segment (start 124.3 93.1) (end 121.4 93.1) (width 1) (layer "F.Cu") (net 2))
 (segment (start 102.7 89.7) (end 103.87 88.53) (width 0.8) (layer "F.Cu") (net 2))
 (segment (start 103.6 88.26) (end 103.87 88.53) (width 0.8) (layer "F.Cu") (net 2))
 (segment (start 134.3 87.2075) (end 129.17 87.2075) (width 3) (layer "F.Cu") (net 2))
 (segment (start 105.6 94.03) (end 103.73 94.03) (width 0.8) (layer "F.Cu") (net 2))
 (segment (start 120.9 89.4) (end 122.2625 88.0375) (width 1) (layer "F.Cu") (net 2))
 (segment (start 110.0125 92.1) (end 110.0125 90.5) (width 0.8) (layer "F.Cu") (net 2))
 (segment (start 129.17 87.2075) (end 129.1 87.1375) (width 1) (layer "F.Cu") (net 2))
 (segment (start 110.5615 90.5) (end 111.9615 89.1) (width 0.4) (layer "F.Cu") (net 2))
 (segment (start 106.33 94.03) (end 105.6 94.03) (width 0.4) (layer "F.Cu") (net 2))
 (segment (start 127.19097 87.2075) (end 125.3 89.09847) (width 1) (layer "F.Cu") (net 2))
 (segment (start 129.17 87.2075) (end 127.19097 87.2075) (width 1) (layer "F.Cu") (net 2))
 (segment (start 118.7 86.6) (end 119 86.9) (width 0.5) (layer "F.Cu") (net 2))
 (segment (start 125.3 92.1) (end 124.3 93.1) (width 1) (layer "F.Cu") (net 2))
 (segment (start 121.4 93.1) (end 120.9 92.6) (width 1) (layer "F.Cu") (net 2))
 (segment (start 112 85.2375) (end 112.2 85.0375) (width 0.4) (layer "F.Cu") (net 2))
 (segment (start 118.7 85.3) (end 118.7 86.6) (width 0.5) (layer "F.Cu") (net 2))
 (segment (start 131.8125 92.4) (end 131.005 91.5925) (width 0.5) (layer "F.Cu") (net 2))
 (segment (start 131.005 91.5925) (end 131.005 89.775) (width 0.5) (layer "F.Cu") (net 2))
 (segment (start 108.6375 85.0375) (end 108.6 85) (width 0.8) (layer "F.Cu") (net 2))
 (segment (start 103.73 94.03) (end 102.7 93) (width 0.8) (layer "F.Cu") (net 2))
 (segment (start 104.5 85) (end 103.6 85.9) (width 1.5) (layer "F.Cu") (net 2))
 (segment (start 111 85.0375) (end 108.6375 85.0375) (width 1.55) (layer "F.Cu") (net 2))
 (segment (start 103.6 85.9) (end 103.6 88.26) (width 1.5) (layer "F.Cu") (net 2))
 (segment (start 110.0125 90.5) (end 110.5615 90.5) (width 0.5) (layer "F.Cu") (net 2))
 (segment (start 124.3375 84.525) (end 124.1125 84.3) (width 1) (layer "F.Cu") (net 6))
 (segment (start 124.3375 86.9) (end 124.3375 87.2625) (width 1) (layer "F.Cu") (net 6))
 (segment (start 128.465 84.5) (end 124.445 84.5) (width 1) (layer "F.Cu") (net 6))
 (segment (start 123.8 88.9) (end 122.7 90) (width 1) (layer "F.Cu") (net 6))
 (segment (start 123.8 87.8) (end 123.8 88.9) (width 1) (layer "F.Cu") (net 6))
 (segment (start 124.3375 86.9) (end 124.3375 84.525) (width 1) (layer "F.Cu") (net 6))
 (segment (start 122.7 90) (end 122.7 91.1) (width 1) (layer "F.Cu") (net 6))
 (segment (start 124.445 86.7925) (end 124.3375 86.9) (width 1) (layer "F.Cu") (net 6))
 (segment (start 124.3375 87.2625) (end 123.8 87.8) (width 1) (layer "F.Cu") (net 6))
 (segment (start 121.9 95.1) (end 120.6 95.1) (width 1) (layer "F.Cu") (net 1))
 (segment (start 118.6 89.134686) (end 119.471128 88.263558) (width 1) (layer "F.Cu") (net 1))
 (segment (start 119.649647 88.15) (end 119.8375 88.15) (width 1) (layer "F.Cu") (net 1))
 (segment (start 120.6 95.1) (end 118.6 93.1) (width 1) (layer "F.Cu") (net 1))
 (segment (start 118.6 93.1) (end 118.6 89.134686) (width 1) (layer "F.Cu") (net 1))
 (segment (start 105.6 91.78) (end 107.8675 91.78) (width 0.4) (layer "F.Cu") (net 14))
 (segment (start 107.8675 91.78) (end 108.1875 92.1) (width 0.4) (layer "F.Cu") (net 14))
 (segment (start 105.6 90.78) (end 107.9075 90.78) (width 0.4) (layer "F.Cu") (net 8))
 (segment (start 107.9075 90.78) (end 108.1875 90.5) (width 0.4) (layer "F.Cu") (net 8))
 (segment (start 126.025 96.2) (end 128.3 96.2) (width 0.5) (layer "F.Cu") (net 16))
 (segment (start 125.5 96.725) (end 126.025 96.2) (width 0.5) (layer "F.Cu") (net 16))
 (segment (start 128.3 96.2) (end 128.8 95.7) (width 0.5) (layer "F.Cu") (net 16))
 (segment (start 120.1125 84.35) (end 120.1125 84.3) (width 0.5) (layer "F.Cu") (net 3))
 (segment (start 120.1125 84.3) (end 122.2875 84.3) (width 0.5) (layer "F.Cu") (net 3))
 (segment (start 119.8375 85.95) (end 119.8375 84.625) (width 0.5) (layer "F.Cu") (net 3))
 (segment (start 119.8375 84.625) (end 120.1125 84.35) (width 0.5) (layer "F.Cu") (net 3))
 (segment (start 129.9875 92.4) (end 129.735 92.1475) (width 0.5) (layer "F.Cu") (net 13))
 (segment (start 129.735 92.1475) (end 129.735 89.775) (width 0.5) (layer "F.Cu") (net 13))
 (segment (start 110.025 93.8125) (end 109.9125 93.7) (width 0.4) (layer "F.Cu") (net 9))
 (segment (start 110.025 95.6) (end 110.025 93.8125) (width 0.4) (layer "F.Cu") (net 9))
 (segment (start 115.5 87.8146) (end 116.2156 87.099) (width 1) (layer "F.Cu") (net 4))
 (segment (start 113.725 88.1625) (end 113.1625 87.6) (width 0.5) (layer "F.Cu") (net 4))
 (segment (start 116.2156 87.099) (end 116.9146 86.4) (width 1) (layer "F.Cu") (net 4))
 (segment (start 115.4 89.9) (end 112.2 93.1) (width 1.5) (layer "F.Cu") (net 4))
 (segment (start 115.5 88.1625) (end 115.4 88.2625) (width 1.5) (layer "F.Cu") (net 4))
 (segment (start 115.5 88.1625) (end 113.725 88.1625) (width 2) (layer "F.Cu") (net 4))
 (segment (start 116.9146 86.4) (end 117.699 86.4) (width 1) (layer "F.Cu") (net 4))
 (segment (start 115.4 88.2625) (end 115.4 89.9) (width 1.5) (layer "F.Cu") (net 4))
 (segment (start 115.5 88.1625) (end 115.5 87.8146) (width 1) (layer "F.Cu") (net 4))
 (segment (start 105.6 89.76) (end 104.24 89.76) (width 0.8) (layer "F.Cu") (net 7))
 (segment (start 104.3 92.8) (end 105.6 92.8) (width 0.8) (layer "F.Cu") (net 7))
 (segment (start 110.8375 87.6) (end 109.1 87.6) (width 1) (layer "F.Cu") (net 7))
 (segment (start 109.1 87.6) (end 106.971 89.729) (width 1) (layer "F.Cu") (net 7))
 (segment (start 104.24 89.76) (end 103.9 90.1) (width 0.8) (layer "F.Cu") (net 7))
 (segment (start 103.9 90.1) (end 103.9 92.4) (width 0.8) (layer "F.Cu") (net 7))
 (segment (start 103.9 92.4) (end 104.3 92.8) (width 0.8) (layer "F.Cu") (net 7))
 (segment (start 107.1875 92.8) (end 105.6 92.8) (width 0.4) (layer "F.Cu") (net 7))
 (segment (start 106.971 89.729) (end 105.6 89.729) (width 1) (layer "F.Cu") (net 7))
 (segment (start 108.0875 93.7) (end 107.1875 92.8) (width 0.4) (layer "F.Cu") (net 7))
 (segment (start 127.195 89.775) (end 127.195 90.495) (width 1) (layer "F.Cu") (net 11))
 (segment (start 127.195 90.495) (end 127.464 90.764) (width 1) (layer "F.Cu") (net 11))
 (segment (start 128.5 91.8) (end 128.5 93.3) (width 1) (layer "F.Cu") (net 11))
 (segment (start 132.6 95.7) (end 132.3075 95.4075) (width 0.5) (layer "F.Cu") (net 11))
 (segment (start 127.9885 91.2885) (end 128.5 91.8) (width 1) (layer "F.Cu") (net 11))
 (segment (start 133.8 95.7) (end 132.6 95.7) (width 0.5) (layer "F.Cu") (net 11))
 (segment (start 127.464 90.794152) (end 127.958348 91.2885) (width 1) (layer "F.Cu") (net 11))
 (segment (start 134.3 91.8075) (end 132.3075 93.8) (width 1) (layer "F.Cu") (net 11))
 (segment (start 127.958348 91.2885) (end 127.9885 91.2885) (width 1) (layer "F.Cu") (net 11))
 (segment (start 132.3075 95.4075) (end 132.3075 93.8) (width 0.5) (layer "F.Cu") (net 11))
 (segment (start 127.464 90.764) (end 127.464 90.794152) (width 1) (layer "F.Cu") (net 11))
 (segment (start 128.5 93.3) (end 129 93.8) (width 1) (layer "F.Cu") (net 11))
 (segment (start 129 93.8) (end 132.3075 93.8) (width 1) (layer "F.Cu") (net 11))
 (segment (start 127.1125 93.0625) (end 125.5 94.675) (width 0.5) (layer "F.Cu") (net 15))
 (segment (start 127.1125 92.4) (end 127.1125 93.0625) (width 0.5) (layer "F.Cu") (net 15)))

